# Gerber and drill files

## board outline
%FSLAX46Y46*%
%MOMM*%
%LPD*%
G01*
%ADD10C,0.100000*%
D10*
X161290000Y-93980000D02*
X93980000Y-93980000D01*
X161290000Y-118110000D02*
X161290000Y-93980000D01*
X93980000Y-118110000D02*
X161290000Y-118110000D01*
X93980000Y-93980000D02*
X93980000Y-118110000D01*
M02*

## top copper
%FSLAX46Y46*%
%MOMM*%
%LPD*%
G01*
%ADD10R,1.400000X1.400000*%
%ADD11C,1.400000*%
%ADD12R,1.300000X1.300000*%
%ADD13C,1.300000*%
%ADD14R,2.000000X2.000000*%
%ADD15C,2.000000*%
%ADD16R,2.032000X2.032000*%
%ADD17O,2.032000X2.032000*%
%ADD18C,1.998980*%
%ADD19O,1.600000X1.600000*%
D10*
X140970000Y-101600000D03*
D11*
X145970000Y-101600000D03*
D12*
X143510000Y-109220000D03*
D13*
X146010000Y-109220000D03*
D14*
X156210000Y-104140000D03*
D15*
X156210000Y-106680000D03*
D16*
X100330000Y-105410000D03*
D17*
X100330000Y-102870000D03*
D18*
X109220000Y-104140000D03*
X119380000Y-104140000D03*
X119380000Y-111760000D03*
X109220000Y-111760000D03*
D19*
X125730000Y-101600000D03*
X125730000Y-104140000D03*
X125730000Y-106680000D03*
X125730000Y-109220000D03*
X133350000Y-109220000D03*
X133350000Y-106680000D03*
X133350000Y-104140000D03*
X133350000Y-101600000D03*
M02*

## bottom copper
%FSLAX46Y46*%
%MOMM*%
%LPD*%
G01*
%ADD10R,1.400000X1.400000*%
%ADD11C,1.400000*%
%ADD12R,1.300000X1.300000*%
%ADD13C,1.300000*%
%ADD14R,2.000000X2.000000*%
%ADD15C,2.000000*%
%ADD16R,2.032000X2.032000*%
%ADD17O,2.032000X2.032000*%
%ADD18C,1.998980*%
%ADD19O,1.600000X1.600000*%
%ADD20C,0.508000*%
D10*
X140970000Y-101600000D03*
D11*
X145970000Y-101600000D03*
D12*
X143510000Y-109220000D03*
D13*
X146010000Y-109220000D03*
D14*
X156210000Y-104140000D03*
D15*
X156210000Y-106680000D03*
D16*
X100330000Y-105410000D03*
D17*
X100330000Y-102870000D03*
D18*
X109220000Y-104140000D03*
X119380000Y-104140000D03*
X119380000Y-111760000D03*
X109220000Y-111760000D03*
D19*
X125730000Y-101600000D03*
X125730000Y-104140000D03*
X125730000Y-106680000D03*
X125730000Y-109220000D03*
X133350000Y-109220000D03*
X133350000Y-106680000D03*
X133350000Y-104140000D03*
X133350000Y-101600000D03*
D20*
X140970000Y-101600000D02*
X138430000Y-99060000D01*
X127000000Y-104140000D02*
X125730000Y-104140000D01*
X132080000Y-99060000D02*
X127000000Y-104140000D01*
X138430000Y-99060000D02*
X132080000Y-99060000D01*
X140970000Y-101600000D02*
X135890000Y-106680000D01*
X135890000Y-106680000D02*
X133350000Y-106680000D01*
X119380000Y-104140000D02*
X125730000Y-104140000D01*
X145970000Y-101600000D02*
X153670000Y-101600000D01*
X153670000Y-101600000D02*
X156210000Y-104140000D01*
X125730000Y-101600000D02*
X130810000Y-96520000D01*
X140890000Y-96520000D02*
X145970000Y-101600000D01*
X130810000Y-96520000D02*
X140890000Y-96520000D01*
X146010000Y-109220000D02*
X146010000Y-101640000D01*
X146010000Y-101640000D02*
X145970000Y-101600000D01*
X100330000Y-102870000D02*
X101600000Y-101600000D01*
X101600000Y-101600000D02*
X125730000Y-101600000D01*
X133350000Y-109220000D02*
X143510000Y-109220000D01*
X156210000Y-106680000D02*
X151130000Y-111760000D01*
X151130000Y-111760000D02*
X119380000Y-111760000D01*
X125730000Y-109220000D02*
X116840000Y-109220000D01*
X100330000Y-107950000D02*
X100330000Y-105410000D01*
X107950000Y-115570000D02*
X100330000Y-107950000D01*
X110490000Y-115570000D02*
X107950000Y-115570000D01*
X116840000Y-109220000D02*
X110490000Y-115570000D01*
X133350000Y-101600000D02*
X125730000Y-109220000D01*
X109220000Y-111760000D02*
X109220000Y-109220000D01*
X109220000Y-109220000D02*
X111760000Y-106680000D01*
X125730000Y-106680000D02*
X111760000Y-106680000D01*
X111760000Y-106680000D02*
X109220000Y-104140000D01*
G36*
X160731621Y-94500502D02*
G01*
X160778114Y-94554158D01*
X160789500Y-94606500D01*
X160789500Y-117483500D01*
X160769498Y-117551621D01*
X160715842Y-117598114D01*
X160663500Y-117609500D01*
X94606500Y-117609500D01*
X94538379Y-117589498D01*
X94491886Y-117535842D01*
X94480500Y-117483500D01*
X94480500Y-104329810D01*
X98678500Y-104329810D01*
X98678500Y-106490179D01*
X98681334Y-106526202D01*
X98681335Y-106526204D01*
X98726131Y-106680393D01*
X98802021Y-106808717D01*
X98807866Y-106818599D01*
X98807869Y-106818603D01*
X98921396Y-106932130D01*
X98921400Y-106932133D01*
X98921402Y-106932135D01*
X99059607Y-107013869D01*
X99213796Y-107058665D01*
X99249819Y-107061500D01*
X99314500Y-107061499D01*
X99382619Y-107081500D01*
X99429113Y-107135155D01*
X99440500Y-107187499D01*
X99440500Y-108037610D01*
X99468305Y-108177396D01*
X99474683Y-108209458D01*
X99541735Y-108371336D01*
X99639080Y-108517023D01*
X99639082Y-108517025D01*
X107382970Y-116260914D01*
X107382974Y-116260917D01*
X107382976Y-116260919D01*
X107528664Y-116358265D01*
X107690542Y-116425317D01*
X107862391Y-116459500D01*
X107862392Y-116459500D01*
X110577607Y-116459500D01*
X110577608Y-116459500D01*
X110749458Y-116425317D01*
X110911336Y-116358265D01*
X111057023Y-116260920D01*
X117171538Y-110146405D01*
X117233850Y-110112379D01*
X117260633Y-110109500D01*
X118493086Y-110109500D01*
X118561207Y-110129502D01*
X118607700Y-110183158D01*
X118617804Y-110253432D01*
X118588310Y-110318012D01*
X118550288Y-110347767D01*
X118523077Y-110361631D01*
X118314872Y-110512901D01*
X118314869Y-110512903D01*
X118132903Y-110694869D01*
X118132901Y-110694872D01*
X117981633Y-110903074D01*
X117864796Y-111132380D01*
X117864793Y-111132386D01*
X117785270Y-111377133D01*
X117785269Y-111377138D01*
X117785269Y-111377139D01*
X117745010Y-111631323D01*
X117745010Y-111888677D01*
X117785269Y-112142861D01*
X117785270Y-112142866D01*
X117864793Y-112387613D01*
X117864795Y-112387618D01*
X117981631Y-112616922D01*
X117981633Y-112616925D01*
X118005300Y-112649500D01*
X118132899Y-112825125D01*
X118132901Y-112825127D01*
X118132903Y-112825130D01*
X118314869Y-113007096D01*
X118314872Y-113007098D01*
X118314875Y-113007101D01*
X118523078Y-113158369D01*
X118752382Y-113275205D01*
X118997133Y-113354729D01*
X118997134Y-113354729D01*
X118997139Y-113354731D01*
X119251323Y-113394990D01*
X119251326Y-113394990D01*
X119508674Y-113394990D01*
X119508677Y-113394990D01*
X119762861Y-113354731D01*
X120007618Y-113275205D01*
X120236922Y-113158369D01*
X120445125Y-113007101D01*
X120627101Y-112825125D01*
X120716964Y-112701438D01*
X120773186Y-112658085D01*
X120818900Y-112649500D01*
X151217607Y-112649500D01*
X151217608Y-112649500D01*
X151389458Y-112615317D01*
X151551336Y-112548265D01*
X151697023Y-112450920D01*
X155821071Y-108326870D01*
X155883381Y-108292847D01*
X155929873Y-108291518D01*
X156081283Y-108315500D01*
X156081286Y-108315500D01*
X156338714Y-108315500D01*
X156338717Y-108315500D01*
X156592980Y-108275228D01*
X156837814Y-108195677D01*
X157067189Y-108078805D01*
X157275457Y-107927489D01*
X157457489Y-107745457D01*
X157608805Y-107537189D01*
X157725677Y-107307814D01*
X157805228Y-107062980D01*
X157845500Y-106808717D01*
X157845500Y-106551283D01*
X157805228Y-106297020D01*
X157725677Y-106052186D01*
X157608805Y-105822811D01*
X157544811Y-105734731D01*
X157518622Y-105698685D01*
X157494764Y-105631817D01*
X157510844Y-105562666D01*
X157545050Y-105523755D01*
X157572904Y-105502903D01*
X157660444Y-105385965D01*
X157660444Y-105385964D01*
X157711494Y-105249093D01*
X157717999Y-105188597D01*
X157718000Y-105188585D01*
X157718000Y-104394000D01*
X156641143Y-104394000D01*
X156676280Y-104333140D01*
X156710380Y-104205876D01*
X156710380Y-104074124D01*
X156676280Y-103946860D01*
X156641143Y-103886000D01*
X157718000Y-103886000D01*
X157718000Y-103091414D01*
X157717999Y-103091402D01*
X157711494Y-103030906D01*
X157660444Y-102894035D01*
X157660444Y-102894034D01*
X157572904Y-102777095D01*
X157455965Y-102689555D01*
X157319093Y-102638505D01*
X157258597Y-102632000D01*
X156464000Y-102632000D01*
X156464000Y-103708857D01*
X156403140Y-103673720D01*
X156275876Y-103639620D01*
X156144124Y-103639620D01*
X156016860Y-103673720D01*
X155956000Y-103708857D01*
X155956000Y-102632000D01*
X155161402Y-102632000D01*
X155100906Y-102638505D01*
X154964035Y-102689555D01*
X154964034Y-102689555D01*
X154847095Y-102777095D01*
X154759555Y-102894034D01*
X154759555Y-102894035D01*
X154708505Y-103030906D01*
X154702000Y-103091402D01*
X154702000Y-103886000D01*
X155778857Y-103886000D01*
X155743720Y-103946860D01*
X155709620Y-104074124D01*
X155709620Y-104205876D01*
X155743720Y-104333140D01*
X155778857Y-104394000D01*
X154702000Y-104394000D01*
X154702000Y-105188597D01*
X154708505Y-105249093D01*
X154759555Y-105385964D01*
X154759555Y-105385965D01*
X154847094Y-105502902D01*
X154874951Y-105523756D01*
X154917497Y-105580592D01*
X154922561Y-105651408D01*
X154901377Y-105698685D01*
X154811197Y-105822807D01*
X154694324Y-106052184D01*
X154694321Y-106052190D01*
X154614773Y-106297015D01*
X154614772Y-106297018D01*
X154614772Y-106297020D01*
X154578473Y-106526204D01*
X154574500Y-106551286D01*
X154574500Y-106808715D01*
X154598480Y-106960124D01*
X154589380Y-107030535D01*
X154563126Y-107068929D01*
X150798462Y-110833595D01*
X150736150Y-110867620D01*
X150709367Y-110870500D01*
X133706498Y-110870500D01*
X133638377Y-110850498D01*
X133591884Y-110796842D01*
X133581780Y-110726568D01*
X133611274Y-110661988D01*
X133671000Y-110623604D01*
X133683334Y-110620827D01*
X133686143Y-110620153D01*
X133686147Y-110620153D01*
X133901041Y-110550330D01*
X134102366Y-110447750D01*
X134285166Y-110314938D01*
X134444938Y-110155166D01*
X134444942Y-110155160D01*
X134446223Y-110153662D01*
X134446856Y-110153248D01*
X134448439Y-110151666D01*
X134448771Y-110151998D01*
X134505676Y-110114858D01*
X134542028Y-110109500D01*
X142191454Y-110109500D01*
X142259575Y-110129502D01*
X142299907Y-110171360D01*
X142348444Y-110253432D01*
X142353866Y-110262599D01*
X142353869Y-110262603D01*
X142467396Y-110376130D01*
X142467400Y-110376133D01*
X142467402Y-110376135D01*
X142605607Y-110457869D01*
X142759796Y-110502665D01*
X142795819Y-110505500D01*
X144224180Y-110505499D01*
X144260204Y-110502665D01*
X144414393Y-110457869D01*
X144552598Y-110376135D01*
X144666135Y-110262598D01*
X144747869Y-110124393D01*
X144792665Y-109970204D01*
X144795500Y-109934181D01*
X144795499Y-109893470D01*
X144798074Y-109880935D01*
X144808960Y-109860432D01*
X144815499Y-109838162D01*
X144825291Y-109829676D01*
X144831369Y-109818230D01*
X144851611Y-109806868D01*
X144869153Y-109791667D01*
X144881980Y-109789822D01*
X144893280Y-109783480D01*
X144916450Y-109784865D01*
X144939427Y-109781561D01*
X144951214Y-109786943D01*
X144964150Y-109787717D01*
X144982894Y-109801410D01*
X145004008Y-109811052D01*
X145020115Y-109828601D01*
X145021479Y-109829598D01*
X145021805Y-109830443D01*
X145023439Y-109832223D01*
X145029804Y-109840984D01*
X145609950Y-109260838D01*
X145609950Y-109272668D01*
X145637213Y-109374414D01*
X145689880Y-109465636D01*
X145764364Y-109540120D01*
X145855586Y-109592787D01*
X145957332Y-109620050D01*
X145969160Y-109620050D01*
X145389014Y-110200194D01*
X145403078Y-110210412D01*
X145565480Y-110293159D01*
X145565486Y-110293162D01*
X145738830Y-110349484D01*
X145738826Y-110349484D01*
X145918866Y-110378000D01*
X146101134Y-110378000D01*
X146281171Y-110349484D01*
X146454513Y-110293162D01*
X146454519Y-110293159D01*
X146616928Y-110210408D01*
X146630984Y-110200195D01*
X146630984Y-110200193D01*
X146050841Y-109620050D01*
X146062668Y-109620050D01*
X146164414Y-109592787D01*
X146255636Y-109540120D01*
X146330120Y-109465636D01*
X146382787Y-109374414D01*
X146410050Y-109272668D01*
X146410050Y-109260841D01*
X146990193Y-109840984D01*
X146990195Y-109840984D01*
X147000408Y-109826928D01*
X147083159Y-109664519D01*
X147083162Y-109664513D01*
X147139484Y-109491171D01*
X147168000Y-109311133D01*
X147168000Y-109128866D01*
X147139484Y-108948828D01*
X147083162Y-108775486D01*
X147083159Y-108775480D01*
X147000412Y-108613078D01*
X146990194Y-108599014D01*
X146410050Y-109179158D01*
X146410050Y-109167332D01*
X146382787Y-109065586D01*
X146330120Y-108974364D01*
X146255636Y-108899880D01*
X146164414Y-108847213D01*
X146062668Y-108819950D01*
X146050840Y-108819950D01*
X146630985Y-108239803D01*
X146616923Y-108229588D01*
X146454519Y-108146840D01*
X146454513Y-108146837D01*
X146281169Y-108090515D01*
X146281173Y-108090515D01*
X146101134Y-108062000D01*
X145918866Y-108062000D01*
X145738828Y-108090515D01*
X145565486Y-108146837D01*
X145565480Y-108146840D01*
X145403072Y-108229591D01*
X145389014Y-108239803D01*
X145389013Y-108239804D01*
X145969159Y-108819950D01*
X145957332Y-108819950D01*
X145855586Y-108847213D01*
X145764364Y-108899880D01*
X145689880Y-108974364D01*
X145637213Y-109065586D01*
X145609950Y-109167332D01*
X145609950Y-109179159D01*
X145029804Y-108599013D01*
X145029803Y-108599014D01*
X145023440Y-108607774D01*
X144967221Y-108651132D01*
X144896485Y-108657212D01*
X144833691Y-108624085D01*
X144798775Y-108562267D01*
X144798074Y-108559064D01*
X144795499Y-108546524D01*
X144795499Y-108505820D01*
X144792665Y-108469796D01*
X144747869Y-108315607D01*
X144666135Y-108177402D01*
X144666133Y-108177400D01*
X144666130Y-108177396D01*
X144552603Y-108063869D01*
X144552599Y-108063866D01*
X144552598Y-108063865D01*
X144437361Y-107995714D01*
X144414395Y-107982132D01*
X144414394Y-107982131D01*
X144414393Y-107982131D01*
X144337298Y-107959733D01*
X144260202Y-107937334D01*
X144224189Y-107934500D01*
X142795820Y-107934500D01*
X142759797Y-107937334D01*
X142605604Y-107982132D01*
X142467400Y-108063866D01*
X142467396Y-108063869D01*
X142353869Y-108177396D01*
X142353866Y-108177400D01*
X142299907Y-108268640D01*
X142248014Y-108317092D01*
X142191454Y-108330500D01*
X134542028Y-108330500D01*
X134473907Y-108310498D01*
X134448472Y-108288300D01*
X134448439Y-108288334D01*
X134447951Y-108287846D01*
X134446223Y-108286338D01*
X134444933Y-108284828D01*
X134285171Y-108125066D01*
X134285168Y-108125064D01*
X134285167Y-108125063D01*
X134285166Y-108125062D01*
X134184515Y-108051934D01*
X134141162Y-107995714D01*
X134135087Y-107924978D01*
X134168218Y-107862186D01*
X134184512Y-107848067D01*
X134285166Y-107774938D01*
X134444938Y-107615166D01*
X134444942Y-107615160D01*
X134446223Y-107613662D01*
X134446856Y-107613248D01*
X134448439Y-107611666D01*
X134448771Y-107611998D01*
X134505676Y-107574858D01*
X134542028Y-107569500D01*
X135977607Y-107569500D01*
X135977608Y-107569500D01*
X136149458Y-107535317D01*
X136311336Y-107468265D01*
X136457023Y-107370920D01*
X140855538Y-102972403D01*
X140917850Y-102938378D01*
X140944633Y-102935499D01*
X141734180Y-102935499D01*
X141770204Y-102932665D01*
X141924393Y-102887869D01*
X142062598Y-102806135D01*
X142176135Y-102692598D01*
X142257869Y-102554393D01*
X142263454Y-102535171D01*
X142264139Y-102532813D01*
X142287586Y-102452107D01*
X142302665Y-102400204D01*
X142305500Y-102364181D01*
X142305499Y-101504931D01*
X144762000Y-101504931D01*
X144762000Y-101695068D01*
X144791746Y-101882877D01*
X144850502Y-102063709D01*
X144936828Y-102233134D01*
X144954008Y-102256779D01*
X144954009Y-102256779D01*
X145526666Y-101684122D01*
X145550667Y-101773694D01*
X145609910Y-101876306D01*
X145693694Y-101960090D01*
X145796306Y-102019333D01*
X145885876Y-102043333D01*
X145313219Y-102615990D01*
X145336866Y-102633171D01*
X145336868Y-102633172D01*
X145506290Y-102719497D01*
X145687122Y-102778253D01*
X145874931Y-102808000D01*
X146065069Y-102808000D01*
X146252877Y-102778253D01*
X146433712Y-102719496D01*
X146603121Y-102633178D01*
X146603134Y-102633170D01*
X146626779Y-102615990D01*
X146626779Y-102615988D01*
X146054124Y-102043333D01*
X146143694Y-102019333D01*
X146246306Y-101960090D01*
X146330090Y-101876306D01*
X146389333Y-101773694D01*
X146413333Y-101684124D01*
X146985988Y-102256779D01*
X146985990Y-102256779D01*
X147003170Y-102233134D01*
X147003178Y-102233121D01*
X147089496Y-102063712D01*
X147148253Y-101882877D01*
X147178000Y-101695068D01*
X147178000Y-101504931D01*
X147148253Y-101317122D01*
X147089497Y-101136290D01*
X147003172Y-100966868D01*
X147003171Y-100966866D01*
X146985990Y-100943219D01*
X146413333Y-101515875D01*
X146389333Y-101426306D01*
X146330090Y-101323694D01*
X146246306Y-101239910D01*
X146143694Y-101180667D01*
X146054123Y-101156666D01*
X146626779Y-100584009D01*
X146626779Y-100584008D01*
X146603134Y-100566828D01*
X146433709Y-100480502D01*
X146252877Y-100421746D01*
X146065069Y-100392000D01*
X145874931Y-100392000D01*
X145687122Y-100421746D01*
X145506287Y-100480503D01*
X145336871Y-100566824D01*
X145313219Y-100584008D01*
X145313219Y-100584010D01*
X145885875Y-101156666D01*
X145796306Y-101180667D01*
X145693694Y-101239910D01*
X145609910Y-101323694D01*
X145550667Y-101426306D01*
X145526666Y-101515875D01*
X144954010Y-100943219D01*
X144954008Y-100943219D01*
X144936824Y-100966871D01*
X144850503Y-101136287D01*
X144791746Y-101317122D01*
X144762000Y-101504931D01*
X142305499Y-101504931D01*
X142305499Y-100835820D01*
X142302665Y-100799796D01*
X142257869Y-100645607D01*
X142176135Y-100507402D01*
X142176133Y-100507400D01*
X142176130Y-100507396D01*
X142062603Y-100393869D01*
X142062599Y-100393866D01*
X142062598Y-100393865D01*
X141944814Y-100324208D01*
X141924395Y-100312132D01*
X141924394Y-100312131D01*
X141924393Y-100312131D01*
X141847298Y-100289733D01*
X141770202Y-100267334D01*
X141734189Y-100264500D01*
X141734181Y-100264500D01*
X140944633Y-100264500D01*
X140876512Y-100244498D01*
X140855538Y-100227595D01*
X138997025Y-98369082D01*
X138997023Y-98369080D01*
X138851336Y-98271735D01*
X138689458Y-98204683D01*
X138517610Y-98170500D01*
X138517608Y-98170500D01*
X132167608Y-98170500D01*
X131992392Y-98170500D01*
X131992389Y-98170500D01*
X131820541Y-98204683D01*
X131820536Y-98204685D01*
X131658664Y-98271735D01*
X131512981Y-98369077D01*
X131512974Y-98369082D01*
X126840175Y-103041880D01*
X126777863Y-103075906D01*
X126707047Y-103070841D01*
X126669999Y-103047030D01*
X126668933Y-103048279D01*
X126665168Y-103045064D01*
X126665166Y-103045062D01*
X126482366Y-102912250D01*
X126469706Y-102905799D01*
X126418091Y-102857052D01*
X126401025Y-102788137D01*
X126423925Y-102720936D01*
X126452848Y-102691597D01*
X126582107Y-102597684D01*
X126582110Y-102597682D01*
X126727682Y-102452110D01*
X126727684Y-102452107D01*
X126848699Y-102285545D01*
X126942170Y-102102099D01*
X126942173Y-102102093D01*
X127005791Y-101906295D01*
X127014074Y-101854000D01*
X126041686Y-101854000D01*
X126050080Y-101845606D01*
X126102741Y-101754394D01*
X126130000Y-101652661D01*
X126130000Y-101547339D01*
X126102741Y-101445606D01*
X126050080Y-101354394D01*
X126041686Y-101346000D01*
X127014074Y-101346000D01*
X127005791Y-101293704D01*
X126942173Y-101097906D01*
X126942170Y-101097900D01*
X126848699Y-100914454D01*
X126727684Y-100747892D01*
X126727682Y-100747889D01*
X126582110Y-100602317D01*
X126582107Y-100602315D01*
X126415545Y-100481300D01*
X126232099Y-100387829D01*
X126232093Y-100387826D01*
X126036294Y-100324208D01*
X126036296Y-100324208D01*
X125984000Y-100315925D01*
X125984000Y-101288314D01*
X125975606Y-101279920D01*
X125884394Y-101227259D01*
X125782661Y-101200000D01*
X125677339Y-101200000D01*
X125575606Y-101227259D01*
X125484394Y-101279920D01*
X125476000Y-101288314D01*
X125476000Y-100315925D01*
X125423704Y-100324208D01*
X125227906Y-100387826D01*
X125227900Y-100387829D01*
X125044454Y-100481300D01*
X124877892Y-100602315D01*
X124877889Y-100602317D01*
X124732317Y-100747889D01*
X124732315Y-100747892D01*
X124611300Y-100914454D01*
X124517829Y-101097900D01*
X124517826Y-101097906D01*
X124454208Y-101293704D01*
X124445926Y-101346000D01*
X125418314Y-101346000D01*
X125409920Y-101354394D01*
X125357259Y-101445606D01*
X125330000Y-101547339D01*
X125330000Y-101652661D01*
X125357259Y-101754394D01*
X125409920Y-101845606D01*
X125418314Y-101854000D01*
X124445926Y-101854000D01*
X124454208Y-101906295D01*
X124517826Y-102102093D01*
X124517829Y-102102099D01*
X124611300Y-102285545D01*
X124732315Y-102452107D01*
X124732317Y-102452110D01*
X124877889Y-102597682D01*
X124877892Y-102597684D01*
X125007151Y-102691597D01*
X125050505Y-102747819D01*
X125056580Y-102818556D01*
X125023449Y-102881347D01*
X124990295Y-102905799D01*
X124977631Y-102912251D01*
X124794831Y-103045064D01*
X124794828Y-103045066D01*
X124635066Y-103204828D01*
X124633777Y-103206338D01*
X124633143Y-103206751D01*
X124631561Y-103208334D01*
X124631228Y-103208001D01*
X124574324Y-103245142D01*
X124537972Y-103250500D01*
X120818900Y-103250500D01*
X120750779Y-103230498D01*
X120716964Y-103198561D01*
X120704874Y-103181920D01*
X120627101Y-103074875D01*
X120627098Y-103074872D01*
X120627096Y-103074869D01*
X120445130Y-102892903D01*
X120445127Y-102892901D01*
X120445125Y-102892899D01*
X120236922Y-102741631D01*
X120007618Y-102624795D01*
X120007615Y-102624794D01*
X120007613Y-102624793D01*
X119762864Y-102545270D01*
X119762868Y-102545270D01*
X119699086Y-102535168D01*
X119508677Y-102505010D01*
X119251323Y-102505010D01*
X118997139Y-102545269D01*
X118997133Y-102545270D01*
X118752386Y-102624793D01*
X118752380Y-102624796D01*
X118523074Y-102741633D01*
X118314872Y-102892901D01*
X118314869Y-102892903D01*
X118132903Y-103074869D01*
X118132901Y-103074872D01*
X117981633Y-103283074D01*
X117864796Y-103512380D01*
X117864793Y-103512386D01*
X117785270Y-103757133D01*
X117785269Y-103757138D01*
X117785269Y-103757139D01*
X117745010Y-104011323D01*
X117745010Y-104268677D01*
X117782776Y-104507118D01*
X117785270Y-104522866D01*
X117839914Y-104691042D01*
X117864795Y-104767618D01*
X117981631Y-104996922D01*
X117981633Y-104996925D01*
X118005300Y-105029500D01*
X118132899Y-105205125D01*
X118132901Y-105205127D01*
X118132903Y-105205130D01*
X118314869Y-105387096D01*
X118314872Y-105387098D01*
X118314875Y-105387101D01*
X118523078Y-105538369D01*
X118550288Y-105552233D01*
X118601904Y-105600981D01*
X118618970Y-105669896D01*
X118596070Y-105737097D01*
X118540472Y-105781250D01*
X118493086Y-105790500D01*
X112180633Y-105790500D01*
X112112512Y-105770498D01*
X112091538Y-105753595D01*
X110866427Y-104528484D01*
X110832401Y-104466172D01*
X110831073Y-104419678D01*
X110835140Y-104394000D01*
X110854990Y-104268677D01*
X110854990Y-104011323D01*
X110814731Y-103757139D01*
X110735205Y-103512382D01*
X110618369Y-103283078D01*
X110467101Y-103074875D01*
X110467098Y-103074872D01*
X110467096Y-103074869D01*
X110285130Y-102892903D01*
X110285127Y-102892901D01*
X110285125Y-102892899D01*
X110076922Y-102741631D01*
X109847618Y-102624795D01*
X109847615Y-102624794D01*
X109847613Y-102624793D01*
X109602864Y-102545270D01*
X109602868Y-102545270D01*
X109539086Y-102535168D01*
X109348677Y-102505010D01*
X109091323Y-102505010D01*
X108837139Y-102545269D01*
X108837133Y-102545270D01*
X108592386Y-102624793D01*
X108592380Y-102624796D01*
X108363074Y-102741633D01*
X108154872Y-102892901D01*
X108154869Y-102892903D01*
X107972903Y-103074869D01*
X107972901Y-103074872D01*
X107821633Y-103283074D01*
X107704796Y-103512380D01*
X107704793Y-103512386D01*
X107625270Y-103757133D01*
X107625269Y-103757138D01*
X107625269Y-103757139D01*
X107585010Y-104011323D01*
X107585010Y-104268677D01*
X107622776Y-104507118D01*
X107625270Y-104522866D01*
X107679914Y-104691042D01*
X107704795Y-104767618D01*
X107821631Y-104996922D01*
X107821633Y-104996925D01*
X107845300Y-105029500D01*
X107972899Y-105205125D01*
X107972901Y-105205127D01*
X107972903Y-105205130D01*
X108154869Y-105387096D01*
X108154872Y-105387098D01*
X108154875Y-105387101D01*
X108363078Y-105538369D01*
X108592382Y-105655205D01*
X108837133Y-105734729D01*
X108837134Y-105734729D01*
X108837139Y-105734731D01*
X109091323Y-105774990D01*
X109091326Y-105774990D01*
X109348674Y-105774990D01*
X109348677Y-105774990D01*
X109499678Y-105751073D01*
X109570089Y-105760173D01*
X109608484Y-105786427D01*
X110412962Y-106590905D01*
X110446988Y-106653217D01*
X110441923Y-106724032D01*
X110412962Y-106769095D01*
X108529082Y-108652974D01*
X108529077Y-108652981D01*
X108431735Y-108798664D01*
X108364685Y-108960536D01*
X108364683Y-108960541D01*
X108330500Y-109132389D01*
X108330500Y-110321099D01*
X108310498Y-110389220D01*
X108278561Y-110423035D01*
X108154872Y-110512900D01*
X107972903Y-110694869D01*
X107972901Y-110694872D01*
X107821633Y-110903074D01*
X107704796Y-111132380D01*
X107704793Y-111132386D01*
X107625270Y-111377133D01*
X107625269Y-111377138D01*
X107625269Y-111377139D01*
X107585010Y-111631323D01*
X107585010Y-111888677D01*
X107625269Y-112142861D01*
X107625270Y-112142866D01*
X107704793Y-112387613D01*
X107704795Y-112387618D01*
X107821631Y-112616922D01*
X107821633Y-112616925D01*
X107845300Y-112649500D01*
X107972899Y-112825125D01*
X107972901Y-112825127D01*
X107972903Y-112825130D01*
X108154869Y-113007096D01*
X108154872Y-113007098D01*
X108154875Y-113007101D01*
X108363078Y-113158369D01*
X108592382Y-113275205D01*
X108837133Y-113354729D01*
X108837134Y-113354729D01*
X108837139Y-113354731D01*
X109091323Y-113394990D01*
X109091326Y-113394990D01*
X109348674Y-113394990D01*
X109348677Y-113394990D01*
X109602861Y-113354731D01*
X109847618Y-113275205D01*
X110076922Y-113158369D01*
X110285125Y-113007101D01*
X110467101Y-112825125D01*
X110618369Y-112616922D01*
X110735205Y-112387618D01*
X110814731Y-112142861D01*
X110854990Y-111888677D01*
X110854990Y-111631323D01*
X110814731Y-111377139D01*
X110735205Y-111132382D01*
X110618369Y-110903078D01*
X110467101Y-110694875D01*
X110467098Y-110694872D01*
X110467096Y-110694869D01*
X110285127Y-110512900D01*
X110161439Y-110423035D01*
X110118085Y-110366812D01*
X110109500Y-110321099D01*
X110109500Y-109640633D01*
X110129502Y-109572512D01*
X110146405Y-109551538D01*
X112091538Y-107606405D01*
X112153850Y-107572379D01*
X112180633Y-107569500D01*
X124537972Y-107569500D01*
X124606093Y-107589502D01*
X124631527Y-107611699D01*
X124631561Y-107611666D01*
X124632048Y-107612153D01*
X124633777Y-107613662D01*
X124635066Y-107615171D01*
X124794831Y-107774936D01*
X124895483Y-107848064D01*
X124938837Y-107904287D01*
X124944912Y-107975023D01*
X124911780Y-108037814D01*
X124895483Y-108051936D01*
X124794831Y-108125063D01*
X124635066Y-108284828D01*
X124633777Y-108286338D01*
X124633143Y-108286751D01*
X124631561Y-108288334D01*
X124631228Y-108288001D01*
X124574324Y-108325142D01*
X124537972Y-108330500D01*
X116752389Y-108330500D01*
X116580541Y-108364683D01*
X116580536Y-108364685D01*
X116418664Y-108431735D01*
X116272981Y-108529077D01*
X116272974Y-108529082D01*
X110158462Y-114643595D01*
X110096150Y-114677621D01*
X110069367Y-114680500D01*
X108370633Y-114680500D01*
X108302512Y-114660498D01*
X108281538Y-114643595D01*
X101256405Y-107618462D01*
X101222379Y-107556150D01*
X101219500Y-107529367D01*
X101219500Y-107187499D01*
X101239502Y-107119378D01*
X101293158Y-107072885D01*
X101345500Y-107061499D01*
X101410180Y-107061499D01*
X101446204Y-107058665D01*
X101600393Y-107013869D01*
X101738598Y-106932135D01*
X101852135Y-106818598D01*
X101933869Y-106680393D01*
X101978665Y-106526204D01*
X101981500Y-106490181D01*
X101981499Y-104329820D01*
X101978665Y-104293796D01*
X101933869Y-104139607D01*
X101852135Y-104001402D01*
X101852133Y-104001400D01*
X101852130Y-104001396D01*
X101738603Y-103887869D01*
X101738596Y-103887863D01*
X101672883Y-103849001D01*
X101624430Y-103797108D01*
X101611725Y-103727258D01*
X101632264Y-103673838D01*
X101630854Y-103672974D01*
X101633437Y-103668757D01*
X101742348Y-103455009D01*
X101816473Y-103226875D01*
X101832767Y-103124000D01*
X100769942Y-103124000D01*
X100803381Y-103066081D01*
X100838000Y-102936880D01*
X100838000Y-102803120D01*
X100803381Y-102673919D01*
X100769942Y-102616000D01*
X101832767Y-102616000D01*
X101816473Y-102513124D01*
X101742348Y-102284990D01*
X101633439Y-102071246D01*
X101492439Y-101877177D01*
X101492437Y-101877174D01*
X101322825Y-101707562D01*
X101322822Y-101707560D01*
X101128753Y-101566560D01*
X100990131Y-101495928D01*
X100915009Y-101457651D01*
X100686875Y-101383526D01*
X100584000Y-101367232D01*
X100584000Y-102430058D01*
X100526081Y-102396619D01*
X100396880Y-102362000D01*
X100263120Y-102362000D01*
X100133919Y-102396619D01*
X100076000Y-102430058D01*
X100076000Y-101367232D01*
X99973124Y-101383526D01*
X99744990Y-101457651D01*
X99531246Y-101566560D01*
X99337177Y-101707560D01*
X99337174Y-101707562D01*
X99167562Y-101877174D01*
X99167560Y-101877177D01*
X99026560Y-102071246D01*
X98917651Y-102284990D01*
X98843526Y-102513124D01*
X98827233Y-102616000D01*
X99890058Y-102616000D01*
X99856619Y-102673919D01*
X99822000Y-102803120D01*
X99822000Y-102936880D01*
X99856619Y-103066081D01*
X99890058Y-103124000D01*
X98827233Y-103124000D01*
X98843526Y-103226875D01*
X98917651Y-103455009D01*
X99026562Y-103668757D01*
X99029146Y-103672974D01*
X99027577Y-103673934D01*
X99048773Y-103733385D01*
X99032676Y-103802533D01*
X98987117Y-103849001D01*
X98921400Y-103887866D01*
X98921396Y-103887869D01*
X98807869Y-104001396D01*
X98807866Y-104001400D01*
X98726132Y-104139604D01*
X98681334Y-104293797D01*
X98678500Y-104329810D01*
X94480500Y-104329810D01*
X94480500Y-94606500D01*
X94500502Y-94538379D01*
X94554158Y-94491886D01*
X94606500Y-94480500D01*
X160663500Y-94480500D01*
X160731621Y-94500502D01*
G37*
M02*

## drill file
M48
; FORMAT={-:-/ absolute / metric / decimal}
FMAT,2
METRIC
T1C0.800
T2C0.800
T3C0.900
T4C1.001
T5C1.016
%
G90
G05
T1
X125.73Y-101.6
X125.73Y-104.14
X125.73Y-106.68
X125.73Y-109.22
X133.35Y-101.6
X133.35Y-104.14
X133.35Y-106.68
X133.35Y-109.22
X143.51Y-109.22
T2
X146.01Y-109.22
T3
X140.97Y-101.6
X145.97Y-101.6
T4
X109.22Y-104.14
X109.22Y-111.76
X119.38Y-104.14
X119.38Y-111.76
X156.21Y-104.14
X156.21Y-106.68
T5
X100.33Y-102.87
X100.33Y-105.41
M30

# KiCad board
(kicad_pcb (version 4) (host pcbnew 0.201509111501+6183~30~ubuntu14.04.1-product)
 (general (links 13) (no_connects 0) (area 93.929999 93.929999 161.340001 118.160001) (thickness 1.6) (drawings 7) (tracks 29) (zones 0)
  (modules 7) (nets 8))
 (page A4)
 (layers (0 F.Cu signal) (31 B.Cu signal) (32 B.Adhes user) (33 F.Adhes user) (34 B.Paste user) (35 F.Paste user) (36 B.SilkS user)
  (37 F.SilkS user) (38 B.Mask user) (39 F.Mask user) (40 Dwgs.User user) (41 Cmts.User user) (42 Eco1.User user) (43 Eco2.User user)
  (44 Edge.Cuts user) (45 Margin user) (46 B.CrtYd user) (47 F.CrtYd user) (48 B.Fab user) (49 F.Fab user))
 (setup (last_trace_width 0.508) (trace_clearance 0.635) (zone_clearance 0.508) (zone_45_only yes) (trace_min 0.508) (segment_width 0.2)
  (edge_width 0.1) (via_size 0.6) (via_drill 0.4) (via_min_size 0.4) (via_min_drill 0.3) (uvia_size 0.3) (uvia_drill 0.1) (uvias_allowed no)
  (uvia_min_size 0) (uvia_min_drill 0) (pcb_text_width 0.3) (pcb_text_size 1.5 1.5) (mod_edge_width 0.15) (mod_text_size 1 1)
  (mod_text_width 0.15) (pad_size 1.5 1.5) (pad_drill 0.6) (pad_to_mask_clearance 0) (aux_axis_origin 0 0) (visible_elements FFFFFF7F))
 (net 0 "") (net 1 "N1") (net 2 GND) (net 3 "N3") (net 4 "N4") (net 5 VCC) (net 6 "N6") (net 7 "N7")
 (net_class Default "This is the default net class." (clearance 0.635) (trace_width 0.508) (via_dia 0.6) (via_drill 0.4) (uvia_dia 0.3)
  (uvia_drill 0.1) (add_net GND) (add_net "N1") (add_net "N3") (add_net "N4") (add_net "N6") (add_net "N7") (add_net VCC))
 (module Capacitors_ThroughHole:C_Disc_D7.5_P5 (layer F.Cu) (at 140.97 101.6)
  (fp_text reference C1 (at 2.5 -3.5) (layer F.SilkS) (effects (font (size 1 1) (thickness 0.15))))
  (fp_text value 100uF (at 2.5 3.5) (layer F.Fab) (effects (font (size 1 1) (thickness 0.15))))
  (pad 1 thru_hole rect (at 0 0) (size 1.4 1.4) (drill 0.9) (layers *.Cu *.Mask F.SilkS) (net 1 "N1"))
  (pad 2 thru_hole circle (at 5 0) (size 1.4 1.4) (drill 0.9) (layers *.Cu *.Mask F.SilkS) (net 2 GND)))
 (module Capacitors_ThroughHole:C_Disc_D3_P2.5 (layer F.Cu) (at 143.51 109.22)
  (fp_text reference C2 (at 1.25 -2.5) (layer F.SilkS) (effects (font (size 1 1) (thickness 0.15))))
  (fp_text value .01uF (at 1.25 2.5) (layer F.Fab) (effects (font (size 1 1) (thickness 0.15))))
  (pad 1 thru_hole rect (at 0 0) (size 1.3 1.3) (drill 0.8) (layers *.Cu *.Mask F.SilkS) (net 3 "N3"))
  (pad 2 thru_hole circle (at 2.5 0) (size 1.3 1.3) (drill 0.8001) (layers *.Cu *.Mask F.SilkS) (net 2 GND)))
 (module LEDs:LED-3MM (layer F.Cu) (at 156.21 104.14 270)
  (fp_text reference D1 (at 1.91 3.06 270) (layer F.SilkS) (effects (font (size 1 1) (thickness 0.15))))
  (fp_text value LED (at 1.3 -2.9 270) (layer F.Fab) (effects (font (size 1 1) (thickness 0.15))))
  (pad 1 thru_hole rect (at 0 0) (size 2 2) (drill 1.00076) (layers *.Cu *.Mask F.SilkS) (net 2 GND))
  (pad 2 thru_hole circle (at 2.54 0 270) (size 2 2) (drill 1.00076) (layers *.Cu *.Mask F.SilkS) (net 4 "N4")))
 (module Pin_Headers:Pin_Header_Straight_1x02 (layer F.Cu) (at 100.33 105.41 180)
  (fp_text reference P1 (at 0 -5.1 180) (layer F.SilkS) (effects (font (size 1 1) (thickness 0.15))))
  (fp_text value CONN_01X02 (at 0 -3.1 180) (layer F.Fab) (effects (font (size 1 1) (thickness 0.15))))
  (pad 1 thru_hole rect (at 0 0 180) (size 2.032 2.032) (drill 1.016) (layers *.Cu *.Mask F.SilkS) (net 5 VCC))
  (pad 2 thru_hole oval (at 0 2.54 180) (size 2.032 2.032) (drill 1.016) (layers *.Cu *.Mask F.SilkS) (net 2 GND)))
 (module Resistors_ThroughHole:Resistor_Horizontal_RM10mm (layer F.Cu) (at 114.3 104.14)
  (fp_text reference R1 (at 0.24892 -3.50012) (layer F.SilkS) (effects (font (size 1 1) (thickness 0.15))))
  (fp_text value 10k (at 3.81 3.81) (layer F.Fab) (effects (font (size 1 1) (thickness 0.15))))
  (pad 1 thru_hole circle (at -5.08 0) (size 1.99898 1.99898) (drill 1.00076) (layers *.Cu *.SilkS *.Mask) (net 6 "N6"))
  (pad 2 thru_hole circle (at 5.08 0) (size 1.99898 1.99898) (drill 1.00076) (layers *.Cu *.SilkS *.Mask) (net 1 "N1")))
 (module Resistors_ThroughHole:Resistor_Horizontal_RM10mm (layer F.Cu) (at 114.3 111.76 180)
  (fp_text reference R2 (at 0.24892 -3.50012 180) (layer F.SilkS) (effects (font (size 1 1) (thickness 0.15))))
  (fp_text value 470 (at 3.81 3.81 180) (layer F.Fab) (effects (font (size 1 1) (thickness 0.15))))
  (pad 1 thru_hole circle (at -5.08 0 180) (size 1.99898 1.99898) (drill 1.00076) (layers *.Cu *.SilkS *.Mask) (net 4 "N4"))
  (pad 2 thru_hole circle (at 5.08 0 180) (size 1.99898 1.99898) (drill 1.00076) (layers *.Cu *.SilkS *.Mask) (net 6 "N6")))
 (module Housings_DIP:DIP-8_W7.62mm (layer F.Cu) (at 125.73 101.6)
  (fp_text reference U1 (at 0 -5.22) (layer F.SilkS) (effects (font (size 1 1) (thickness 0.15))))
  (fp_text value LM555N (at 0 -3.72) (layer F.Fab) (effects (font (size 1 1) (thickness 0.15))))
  (pad 1 thru_hole oval (at 0 0) (size 1.6 1.6) (drill 0.8) (layers *.Cu *.Mask F.SilkS) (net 2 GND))
  (pad 2 thru_hole oval (at 0 2.54) (size 1.6 1.6) (drill 0.8) (layers *.Cu *.Mask F.SilkS) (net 1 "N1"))
  (pad 3 thru_hole oval (at 0 5.08) (size 1.6 1.6) (drill 0.8) (layers *.Cu *.Mask F.SilkS) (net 6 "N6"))
  (pad 4 thru_hole oval (at 0 7.62) (size 1.6 1.6) (drill 0.8) (layers *.Cu *.Mask F.SilkS) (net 5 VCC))
  (pad 5 thru_hole oval (at 7.62 7.62) (size 1.6 1.6) (drill 0.8) (layers *.Cu *.Mask F.SilkS) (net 3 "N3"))
  (pad 6 thru_hole oval (at 7.62 5.08) (size 1.6 1.6) (drill 0.8) (layers *.Cu *.Mask F.SilkS) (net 1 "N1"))
  (pad 7 thru_hole oval (at 7.62 2.54) (size 1.6 1.6) (drill 0.8) (layers *.Cu *.Mask F.SilkS) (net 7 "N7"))
  (pad 8 thru_hole oval (at 7.62 0) (size 1.6 1.6) (drill 0.8) (layers *.Cu *.Mask F.SilkS) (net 5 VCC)))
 (gr_line (start 161.29 93.98) (end 93.98 93.98) (angle 90) (layer Edge.Cuts) (width 0.1))
 (gr_line (start 161.29 118.11) (end 161.29 93.98) (angle 90) (layer Edge.Cuts) (width 0.1))
 (gr_line (start 93.98 118.11) (end 161.29 118.11) (angle 90) (layer Edge.Cuts) (width 0.1))
 (gr_line (start 93.98 93.98) (end 93.98 118.11) (angle 90) (layer Edge.Cuts) (width 0.1))
 (segment (start 140.97 101.6) (end 138.43 99.06) (width 0.508) (layer B.Cu) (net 1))
 (segment (start 127 104.14) (end 125.73 104.14) (width 0.508) (layer B.Cu) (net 1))
 (segment (start 132.08 99.06) (end 127 104.14) (width 0.508) (layer B.Cu) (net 1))
 (segment (start 138.43 99.06) (end 132.08 99.06) (width 0.508) (layer B.Cu) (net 1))
 (segment (start 140.97 101.6) (end 135.89 106.68) (width 0.508) (layer B.Cu) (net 1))
 (segment (start 135.89 106.68) (end 133.35 106.68) (width 0.508) (layer B.Cu) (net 1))
 (segment (start 119.38 104.14) (end 125.73 104.14) (width 0.508) (layer B.Cu) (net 1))
 (segment (start 145.97 101.6) (end 153.67 101.6) (width 0.508) (layer B.Cu) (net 2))
 (segment (start 153.67 101.6) (end 156.21 104.14) (width 0.508) (layer B.Cu) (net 2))
 (segment (start 125.73 101.6) (end 130.81 96.52) (width 0.508) (layer B.Cu) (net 2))
 (segment (start 140.89 96.52) (end 145.97 101.6) (width 0.508) (layer B.Cu) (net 2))
 (segment (start 130.81 96.52) (end 140.89 96.52) (width 0.508) (layer B.Cu) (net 2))
 (segment (start 146.01 109.22) (end 146.01 101.64) (width 0.508) (layer B.Cu) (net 2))
 (segment (start 146.01 101.64) (end 145.97 101.6) (width 0.508) (layer B.Cu) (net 2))
 (segment (start 100.33 102.87) (end 101.6 101.6) (width 0.508) (layer B.Cu) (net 2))
 (segment (start 101.6 101.6) (end 125.73 101.6) (width 0.508) (layer B.Cu) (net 2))
 (segment (start 133.35 109.22) (end 143.51 109.22) (width 0.508) (layer B.Cu) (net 3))
 (segment (start 156.21 106.68) (end 151.13 111.76) (width 0.508) (layer B.Cu) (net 4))
 (segment (start 151.13 111.76) (end 119.38 111.76) (width 0.508) (layer B.Cu) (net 4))
 (segment (start 125.73 109.22) (end 116.84 109.22) (width 0.508) (layer B.Cu) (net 5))
 (segment (start 100.33 107.95) (end 100.33 105.41) (width 0.508) (layer B.Cu) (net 5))
 (segment (start 107.95 115.57) (end 100.33 107.95) (width 0.508) (layer B.Cu) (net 5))
 (segment (start 110.49 115.57) (end 107.95 115.57) (width 0.508) (layer B.Cu) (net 5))
 (segment (start 116.84 109.22) (end 110.49 115.57) (width 0.508) (layer B.Cu) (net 5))
 (segment (start 133.35 101.6) (end 125.73 109.22) (width 0.508) (layer B.Cu) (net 5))
 (segment (start 109.22 111.76) (end 109.22 109.22) (width 0.508) (layer B.Cu) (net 6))
 (segment (start 109.22 109.22) (end 111.76 106.68) (width 0.508) (layer B.Cu) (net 6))
 (segment (start 125.73 106.68) (end 111.76 106.68) (width 0.508) (layer B.Cu) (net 6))
 (segment (start 111.76 106.68) (end 109.22 104.14) (width 0.508) (layer B.Cu) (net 6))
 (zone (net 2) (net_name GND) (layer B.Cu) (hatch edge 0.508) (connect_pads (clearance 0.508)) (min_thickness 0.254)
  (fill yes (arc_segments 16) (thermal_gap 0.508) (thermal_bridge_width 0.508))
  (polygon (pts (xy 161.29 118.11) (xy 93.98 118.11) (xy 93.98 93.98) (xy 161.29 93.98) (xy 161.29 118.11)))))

